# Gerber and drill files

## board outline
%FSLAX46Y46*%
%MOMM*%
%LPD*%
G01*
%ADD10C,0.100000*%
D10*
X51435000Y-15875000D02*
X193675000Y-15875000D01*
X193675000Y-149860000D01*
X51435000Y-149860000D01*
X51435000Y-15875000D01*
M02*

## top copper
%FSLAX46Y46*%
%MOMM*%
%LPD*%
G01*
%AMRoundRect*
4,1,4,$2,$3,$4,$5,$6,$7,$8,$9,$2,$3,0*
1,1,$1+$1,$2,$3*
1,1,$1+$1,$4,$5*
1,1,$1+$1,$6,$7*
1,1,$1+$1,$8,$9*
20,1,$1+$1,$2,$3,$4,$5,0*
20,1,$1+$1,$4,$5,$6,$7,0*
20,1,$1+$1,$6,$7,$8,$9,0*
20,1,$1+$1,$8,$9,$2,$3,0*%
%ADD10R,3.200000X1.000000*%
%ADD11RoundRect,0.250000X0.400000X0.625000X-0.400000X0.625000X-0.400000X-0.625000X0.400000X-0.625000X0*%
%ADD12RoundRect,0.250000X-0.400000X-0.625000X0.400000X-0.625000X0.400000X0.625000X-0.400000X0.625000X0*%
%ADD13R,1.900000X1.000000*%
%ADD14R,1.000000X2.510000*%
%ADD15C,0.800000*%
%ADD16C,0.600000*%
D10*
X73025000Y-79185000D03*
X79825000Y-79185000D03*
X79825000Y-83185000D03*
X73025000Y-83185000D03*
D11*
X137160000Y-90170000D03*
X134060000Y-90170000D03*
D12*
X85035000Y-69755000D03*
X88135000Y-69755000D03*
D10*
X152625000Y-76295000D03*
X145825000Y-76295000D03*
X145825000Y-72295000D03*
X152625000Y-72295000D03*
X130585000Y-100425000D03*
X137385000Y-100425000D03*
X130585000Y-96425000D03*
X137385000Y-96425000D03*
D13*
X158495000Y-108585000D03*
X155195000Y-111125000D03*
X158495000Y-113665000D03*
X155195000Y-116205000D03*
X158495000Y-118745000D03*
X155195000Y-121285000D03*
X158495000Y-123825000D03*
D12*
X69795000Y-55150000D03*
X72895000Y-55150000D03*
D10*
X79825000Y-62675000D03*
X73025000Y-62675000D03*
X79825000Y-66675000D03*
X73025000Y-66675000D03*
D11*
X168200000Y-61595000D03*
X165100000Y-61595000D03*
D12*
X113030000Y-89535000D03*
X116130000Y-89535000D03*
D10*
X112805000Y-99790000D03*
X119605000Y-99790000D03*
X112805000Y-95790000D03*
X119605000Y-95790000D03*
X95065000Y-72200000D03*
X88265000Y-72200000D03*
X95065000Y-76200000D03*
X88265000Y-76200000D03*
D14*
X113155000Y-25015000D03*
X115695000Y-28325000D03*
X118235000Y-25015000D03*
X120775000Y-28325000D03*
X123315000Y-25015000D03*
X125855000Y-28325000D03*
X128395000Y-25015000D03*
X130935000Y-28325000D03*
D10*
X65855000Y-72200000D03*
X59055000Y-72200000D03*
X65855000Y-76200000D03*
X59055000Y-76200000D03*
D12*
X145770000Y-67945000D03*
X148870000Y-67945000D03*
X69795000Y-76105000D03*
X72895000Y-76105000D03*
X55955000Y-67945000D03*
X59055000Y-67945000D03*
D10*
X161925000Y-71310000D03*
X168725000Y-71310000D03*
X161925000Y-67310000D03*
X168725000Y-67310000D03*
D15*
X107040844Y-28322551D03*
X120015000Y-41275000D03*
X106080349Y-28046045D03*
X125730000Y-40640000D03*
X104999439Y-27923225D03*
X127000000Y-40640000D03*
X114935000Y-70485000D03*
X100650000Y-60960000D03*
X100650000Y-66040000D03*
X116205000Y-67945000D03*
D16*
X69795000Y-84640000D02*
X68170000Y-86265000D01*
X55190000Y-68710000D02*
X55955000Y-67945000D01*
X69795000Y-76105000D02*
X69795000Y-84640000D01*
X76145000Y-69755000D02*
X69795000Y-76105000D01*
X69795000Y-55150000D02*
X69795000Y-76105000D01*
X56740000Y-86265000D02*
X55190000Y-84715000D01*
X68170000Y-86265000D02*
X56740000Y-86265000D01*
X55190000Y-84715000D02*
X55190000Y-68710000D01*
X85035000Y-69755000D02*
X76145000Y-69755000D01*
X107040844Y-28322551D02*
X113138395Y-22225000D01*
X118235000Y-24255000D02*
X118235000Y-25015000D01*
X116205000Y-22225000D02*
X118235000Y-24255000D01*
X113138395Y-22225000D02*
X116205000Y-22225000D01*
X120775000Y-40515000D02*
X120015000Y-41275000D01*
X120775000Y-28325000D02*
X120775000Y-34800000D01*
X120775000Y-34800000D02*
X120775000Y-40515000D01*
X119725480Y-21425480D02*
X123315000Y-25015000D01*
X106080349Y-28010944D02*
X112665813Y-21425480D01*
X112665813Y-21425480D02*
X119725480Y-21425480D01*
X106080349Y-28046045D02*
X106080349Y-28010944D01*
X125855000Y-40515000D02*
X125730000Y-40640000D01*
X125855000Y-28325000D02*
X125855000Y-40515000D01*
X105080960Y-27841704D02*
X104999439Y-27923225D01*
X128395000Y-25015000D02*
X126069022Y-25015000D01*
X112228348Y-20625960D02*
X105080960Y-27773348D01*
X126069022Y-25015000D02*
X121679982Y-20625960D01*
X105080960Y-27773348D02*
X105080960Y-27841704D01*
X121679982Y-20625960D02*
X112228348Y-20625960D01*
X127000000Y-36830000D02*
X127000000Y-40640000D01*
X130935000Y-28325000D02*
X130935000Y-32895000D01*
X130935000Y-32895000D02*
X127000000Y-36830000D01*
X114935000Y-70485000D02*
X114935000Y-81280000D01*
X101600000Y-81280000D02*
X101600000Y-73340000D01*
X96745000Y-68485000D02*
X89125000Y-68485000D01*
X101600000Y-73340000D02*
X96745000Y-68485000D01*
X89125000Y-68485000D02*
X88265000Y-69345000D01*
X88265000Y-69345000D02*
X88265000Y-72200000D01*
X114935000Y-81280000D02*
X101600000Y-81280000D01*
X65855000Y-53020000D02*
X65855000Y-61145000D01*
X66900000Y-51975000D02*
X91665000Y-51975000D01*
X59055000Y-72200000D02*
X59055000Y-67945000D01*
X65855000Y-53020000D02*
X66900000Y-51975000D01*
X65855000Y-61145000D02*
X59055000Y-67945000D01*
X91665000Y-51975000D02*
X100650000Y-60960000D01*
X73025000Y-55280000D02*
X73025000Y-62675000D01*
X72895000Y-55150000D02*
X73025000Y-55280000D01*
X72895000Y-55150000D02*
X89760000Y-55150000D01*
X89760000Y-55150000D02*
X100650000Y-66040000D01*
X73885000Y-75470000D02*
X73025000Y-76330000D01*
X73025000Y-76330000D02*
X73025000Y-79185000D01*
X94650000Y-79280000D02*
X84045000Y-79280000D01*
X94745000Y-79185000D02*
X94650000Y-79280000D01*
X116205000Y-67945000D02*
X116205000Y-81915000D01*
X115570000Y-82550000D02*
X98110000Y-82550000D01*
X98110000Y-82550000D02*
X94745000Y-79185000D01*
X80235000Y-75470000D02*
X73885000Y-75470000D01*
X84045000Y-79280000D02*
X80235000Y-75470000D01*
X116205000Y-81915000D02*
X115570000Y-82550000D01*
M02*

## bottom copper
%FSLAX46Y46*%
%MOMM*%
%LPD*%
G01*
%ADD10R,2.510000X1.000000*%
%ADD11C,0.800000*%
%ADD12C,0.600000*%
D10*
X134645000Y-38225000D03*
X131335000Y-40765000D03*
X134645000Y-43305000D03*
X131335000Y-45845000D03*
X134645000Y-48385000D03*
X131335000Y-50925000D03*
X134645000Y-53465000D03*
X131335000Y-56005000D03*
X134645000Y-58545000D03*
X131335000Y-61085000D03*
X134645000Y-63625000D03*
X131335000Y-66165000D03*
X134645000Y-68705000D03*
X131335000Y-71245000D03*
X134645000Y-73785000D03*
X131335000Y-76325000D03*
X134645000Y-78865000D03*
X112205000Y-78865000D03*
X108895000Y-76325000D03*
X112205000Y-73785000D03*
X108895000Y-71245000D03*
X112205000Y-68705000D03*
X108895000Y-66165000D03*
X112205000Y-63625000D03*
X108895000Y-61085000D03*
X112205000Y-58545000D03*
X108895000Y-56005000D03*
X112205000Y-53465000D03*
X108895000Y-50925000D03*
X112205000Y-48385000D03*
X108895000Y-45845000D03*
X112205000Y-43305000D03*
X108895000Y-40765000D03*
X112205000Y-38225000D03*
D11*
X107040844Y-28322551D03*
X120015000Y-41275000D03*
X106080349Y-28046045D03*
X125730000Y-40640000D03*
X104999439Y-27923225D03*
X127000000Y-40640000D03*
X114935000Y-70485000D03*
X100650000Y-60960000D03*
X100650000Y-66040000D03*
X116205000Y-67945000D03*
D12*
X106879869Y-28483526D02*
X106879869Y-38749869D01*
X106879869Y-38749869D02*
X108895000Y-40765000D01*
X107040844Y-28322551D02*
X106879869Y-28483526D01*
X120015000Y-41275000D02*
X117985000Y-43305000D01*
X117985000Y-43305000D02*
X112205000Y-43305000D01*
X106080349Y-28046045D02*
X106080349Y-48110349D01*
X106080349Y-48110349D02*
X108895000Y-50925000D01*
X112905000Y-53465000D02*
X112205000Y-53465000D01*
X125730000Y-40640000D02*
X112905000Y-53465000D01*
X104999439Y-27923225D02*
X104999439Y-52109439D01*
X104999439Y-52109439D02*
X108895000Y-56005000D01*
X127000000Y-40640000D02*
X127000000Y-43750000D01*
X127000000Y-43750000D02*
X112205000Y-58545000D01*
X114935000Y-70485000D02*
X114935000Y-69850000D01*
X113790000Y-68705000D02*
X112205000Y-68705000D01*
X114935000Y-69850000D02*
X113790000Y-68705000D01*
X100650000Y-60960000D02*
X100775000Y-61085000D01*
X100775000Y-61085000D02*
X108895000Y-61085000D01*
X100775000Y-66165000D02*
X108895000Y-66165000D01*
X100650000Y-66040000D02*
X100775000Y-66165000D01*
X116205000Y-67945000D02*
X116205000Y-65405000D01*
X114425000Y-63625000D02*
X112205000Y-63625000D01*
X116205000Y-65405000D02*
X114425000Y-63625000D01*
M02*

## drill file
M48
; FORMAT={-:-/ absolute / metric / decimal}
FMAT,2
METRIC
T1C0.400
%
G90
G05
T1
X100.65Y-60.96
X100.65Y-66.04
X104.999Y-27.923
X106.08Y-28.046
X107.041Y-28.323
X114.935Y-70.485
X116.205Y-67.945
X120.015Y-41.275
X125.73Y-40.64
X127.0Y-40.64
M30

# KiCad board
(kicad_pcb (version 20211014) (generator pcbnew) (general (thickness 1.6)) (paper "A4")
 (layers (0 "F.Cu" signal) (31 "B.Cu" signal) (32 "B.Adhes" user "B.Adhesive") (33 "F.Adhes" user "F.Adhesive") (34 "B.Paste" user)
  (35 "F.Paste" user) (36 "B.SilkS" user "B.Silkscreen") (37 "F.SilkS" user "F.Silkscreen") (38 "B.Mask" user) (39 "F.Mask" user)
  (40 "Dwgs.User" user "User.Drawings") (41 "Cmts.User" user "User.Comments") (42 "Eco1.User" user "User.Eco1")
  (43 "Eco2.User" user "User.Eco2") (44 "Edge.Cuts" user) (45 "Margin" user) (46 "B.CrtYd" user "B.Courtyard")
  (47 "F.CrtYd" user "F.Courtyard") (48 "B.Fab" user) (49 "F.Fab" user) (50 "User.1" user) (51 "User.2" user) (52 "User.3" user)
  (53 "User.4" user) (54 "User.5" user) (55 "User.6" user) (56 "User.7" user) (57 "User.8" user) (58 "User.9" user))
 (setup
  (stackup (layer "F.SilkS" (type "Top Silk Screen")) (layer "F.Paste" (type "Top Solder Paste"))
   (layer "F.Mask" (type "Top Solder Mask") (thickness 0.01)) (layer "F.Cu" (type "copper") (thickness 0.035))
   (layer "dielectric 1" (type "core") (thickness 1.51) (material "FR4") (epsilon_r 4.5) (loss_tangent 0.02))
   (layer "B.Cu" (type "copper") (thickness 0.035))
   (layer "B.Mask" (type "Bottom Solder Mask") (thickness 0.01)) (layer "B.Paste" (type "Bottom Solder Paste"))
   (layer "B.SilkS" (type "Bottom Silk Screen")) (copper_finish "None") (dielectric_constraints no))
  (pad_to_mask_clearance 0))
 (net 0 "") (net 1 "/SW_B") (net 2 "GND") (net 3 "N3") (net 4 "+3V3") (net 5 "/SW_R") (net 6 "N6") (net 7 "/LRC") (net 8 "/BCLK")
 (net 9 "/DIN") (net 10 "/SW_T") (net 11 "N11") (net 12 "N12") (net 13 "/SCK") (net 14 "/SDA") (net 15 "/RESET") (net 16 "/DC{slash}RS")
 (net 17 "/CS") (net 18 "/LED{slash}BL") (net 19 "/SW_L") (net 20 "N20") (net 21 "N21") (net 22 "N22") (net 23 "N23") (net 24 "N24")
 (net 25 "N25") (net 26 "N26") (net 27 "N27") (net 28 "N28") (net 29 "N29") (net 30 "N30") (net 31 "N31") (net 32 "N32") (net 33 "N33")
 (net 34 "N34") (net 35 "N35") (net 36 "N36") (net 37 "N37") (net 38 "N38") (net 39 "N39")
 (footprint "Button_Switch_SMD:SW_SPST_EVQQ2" (layer "F.Cu") (at 76.425 81.185)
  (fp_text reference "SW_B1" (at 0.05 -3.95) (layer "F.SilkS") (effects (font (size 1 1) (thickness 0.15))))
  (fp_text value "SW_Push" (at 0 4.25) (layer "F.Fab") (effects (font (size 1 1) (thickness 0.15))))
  (pad "1" smd rect (at -3.4 -2) (size 3.2 1) (layers "F.Cu" "F.Paste" "F.Mask") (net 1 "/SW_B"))
  (pad "1" smd rect (at 3.4 -2) (size 3.2 1) (layers "F.Cu" "F.Paste" "F.Mask") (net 1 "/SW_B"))
  (pad "2" smd rect (at 3.4 2) (size 3.2 1) (layers "F.Cu" "F.Paste" "F.Mask") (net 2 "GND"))
  (pad "2" smd rect (at -3.4 2) (size 3.2 1) (layers "F.Cu" "F.Paste" "F.Mask") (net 2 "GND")))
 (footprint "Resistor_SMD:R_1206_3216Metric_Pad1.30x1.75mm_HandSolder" (layer "F.Cu") (at 135.61 90.17 180)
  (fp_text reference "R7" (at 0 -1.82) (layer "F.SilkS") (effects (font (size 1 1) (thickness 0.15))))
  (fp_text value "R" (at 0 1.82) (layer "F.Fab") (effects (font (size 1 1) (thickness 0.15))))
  (pad "1" smd roundrect (at -1.55 0 180) (size 1.3 1.75) (layers "F.Cu" "F.Paste" "F.Mask") (roundrect_rratio 0.192308) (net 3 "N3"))
  (pad "2" smd roundrect (at 1.55 0 180) (size 1.3 1.75) (layers "F.Cu" "F.Paste" "F.Mask") (roundrect_rratio 0.192308) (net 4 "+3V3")))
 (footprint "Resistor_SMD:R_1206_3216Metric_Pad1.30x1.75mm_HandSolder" (layer "F.Cu") (at 86.585 69.755)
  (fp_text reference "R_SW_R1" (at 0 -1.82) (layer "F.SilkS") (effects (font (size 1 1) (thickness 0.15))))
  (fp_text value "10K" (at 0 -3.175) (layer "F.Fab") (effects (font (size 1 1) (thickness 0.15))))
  (pad "1" smd roundrect (at -1.55 0) (size 1.3 1.75) (layers "F.Cu" "F.Paste" "F.Mask") (roundrect_rratio 0.192308) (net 4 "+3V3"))
  (pad "2" smd roundrect (at 1.55 0) (size 1.3 1.75) (layers "F.Cu" "F.Paste" "F.Mask") (roundrect_rratio 0.192308) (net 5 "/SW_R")))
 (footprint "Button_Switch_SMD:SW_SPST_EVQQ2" (layer "F.Cu") (at 149.225 74.295 180)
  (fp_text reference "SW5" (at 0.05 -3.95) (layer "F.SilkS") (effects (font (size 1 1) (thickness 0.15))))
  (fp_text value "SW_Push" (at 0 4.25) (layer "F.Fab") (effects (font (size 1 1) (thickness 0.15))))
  (pad "1" smd rect (at -3.4 -2 180) (size 3.2 1) (layers "F.Cu" "F.Paste" "F.Mask") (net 2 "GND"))
  (pad "1" smd rect (at 3.4 -2 180) (size 3.2 1) (layers "F.Cu" "F.Paste" "F.Mask") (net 2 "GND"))
  (pad "2" smd rect (at 3.4 2 180) (size 3.2 1) (layers "F.Cu" "F.Paste" "F.Mask") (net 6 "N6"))
  (pad "2" smd rect (at -3.4 2 180) (size 3.2 1) (layers "F.Cu" "F.Paste" "F.Mask") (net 6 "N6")))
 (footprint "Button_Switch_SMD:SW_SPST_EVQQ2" (layer "F.Cu") (at 133.985 98.425 180)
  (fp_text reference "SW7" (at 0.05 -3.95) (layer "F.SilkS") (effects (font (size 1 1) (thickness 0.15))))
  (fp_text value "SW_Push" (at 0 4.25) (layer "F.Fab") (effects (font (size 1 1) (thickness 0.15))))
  (pad "1" smd rect (at 3.4 -2 180) (size 3.2 1) (layers "F.Cu" "F.Paste" "F.Mask") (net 2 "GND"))
  (pad "1" smd rect (at -3.4 -2 180) (size 3.2 1) (layers "F.Cu" "F.Paste" "F.Mask") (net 2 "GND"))
  (pad "2" smd rect (at 3.4 2 180) (size 3.2 1) (layers "F.Cu" "F.Paste" "F.Mask") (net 3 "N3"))
  (pad "2" smd rect (at -3.4 2 180) (size 3.2 1) (layers "F.Cu" "F.Paste" "F.Mask") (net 3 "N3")))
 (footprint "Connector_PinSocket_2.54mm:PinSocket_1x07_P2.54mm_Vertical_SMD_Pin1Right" (layer "F.Cu") (at 156.845 116.205)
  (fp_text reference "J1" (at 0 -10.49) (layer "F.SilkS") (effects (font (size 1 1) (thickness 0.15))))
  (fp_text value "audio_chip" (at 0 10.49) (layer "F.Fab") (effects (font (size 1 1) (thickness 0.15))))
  (pad "1" smd rect (at 1.65 -7.62) (size 1.9 1) (layers "F.Cu" "F.Paste" "F.Mask") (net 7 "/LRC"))
  (pad "2" smd rect (at -1.65 -5.08) (size 1.9 1) (layers "F.Cu" "F.Paste" "F.Mask") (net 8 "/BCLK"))
  (pad "3" smd rect (at 1.65 -2.54) (size 1.9 1) (layers "F.Cu" "F.Paste" "F.Mask") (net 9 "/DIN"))
  (pad "4" smd rect (at -1.65 0) (size 1.9 1) (layers "F.Cu" "F.Paste" "F.Mask") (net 2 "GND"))
  (pad "5" smd rect (at 1.65 2.54) (size 1.9 1) (layers "F.Cu" "F.Paste" "F.Mask") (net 2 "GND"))
  (pad "6" smd rect (at -1.65 5.08) (size 1.9 1) (layers "F.Cu" "F.Paste" "F.Mask") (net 2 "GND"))
  (pad "7" smd rect (at 1.65 7.62) (size 1.9 1) (layers "F.Cu" "F.Paste" "F.Mask") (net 4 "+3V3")))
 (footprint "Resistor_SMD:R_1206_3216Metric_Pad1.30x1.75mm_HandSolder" (layer "F.Cu") (at 71.345 55.15)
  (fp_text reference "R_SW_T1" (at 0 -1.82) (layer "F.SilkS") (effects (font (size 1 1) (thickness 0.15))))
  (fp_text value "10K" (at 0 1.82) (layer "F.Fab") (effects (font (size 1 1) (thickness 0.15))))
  (pad "1" smd roundrect (at -1.55 0) (size 1.3 1.75) (layers "F.Cu" "F.Paste" "F.Mask") (roundrect_rratio 0.192308) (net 4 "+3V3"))
  (pad "2" smd roundrect (at 1.55 0) (size 1.3 1.75) (layers "F.Cu" "F.Paste" "F.Mask") (roundrect_rratio 0.192308) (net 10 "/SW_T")))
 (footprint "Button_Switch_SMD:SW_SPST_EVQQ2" (layer "F.Cu") (at 76.425 64.675)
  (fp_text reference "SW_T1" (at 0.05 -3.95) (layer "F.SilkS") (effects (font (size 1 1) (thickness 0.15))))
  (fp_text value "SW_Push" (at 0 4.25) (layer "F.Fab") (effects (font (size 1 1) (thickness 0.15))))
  (pad "1" smd rect (at 3.4 -2) (size 3.2 1) (layers "F.Cu" "F.Paste" "F.Mask") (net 10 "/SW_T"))
  (pad "1" smd rect (at -3.4 -2) (size 3.2 1) (layers "F.Cu" "F.Paste" "F.Mask") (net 10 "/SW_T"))
  (pad "2" smd rect (at 3.4 2) (size 3.2 1) (layers "F.Cu" "F.Paste" "F.Mask") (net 2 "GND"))
  (pad "2" smd rect (at -3.4 2) (size 3.2 1) (layers "F.Cu" "F.Paste" "F.Mask") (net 2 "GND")))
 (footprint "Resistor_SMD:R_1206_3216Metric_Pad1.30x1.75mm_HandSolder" (layer "F.Cu") (at 166.65 61.595 180)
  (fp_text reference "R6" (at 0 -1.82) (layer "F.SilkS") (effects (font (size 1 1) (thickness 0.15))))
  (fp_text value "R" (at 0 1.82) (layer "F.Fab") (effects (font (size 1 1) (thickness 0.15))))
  (pad "1" smd roundrect (at -1.55 0 180) (size 1.3 1.75) (layers "F.Cu" "F.Paste" "F.Mask") (roundrect_rratio 0.192308) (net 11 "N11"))
  (pad "2" smd roundrect (at 1.55 0 180) (size 1.3 1.75) (layers "F.Cu" "F.Paste" "F.Mask") (roundrect_rratio 0.192308) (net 4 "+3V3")))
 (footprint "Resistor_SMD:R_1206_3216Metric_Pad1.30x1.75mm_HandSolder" (layer "F.Cu") (at 114.58 89.535)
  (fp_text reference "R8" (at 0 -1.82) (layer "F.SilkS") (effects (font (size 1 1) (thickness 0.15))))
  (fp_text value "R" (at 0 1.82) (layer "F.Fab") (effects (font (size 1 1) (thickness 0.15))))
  (pad "1" smd roundrect (at -1.55 0) (size 1.3 1.75) (layers "F.Cu" "F.Paste" "F.Mask") (roundrect_rratio 0.192308) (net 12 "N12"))
  (pad "2" smd roundrect (at 1.55 0) (size 1.3 1.75) (layers "F.Cu" "F.Paste" "F.Mask") (roundrect_rratio 0.192308) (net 4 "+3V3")))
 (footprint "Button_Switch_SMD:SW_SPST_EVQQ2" (layer "F.Cu") (at 116.205 97.79 180)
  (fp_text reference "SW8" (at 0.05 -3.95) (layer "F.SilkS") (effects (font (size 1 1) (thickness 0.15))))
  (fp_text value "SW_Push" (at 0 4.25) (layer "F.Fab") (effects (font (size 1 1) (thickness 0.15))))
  (pad "1" smd rect (at 3.4 -2 180) (size 3.2 1) (layers "F.Cu" "F.Paste" "F.Mask") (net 2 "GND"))
  (pad "1" smd rect (at -3.4 -2 180) (size 3.2 1) (layers "F.Cu" "F.Paste" "F.Mask") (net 2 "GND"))
  (pad "2" smd rect (at 3.4 2 180) (size 3.2 1) (layers "F.Cu" "F.Paste" "F.Mask") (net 12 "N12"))
  (pad "2" smd rect (at -3.4 2 180) (size 3.2 1) (layers "F.Cu" "F.Paste" "F.Mask") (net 12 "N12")))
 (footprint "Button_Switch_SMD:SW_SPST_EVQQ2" (layer "F.Cu") (at 91.665 74.2)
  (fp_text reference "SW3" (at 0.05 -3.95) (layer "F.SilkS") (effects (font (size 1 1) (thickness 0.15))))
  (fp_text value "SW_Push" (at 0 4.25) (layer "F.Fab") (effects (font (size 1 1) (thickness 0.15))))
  (pad "1" smd rect (at 3.4 -2) (size 3.2 1) (layers "F.Cu" "F.Paste" "F.Mask") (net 5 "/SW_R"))
  (pad "1" smd rect (at -3.4 -2) (size 3.2 1) (layers "F.Cu" "F.Paste" "F.Mask") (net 5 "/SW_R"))
  (pad "2" smd rect (at 3.4 2) (size 3.2 1) (layers "F.Cu" "F.Paste" "F.Mask") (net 2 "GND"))
  (pad "2" smd rect (at -3.4 2) (size 3.2 1) (layers "F.Cu" "F.Paste" "F.Mask") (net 2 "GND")))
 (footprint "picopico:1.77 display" (layer "F.Cu") (at 121.92 22.86 90)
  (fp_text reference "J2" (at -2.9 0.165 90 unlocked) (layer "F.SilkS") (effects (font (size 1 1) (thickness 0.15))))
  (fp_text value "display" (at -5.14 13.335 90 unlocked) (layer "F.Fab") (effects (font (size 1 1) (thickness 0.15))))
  (pad "1" smd rect (at -2.155 -8.765 90) (size 2.51 1) (layers "F.Cu" "F.Paste" "F.Mask") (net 2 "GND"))
  (pad "2" smd rect (at -5.465 -6.225 90) (size 2.51 1) (layers "F.Cu" "F.Paste" "F.Mask") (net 4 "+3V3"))
  (pad "3" smd rect (at -2.155 -3.685 90) (size 2.51 1) (layers "F.Cu" "F.Paste" "F.Mask") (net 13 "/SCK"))
  (pad "4" smd rect (at -5.465 -1.145 90) (size 2.51 1) (layers "F.Cu" "F.Paste" "F.Mask") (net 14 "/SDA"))
  (pad "5" smd rect (at -2.155 1.395 90) (size 2.51 1) (layers "F.Cu" "F.Paste" "F.Mask") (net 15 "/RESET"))
  (pad "6" smd rect (at -5.465 3.935 90) (size 2.51 1) (layers "F.Cu" "F.Paste" "F.Mask") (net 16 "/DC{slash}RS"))
  (pad "7" smd rect (at -2.155 6.475 90) (size 2.51 1) (layers "F.Cu" "F.Paste" "F.Mask") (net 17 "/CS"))
  (pad "8" smd rect (at -5.465 9.015 90) (size 2.51 1) (layers "F.Cu" "F.Paste" "F.Mask") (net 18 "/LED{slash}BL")))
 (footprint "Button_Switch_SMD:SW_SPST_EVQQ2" (layer "F.Cu") (at 62.455 74.2)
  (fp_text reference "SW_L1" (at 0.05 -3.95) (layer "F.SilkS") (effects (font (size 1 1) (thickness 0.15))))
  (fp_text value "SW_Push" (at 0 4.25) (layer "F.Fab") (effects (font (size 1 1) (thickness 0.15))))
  (pad "1" smd rect (at 3.4 -2) (size 3.2 1) (layers "F.Cu" "F.Paste" "F.Mask") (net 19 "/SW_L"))
  (pad "1" smd rect (at -3.4 -2) (size 3.2 1) (layers "F.Cu" "F.Paste" "F.Mask") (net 19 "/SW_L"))
  (pad "2" smd rect (at 3.4 2) (size 3.2 1) (layers "F.Cu" "F.Paste" "F.Mask") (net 2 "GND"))
  (pad "2" smd rect (at -3.4 2) (size 3.2 1) (layers "F.Cu" "F.Paste" "F.Mask") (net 2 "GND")))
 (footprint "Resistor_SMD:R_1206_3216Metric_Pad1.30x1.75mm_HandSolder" (layer "F.Cu") (at 147.32 67.945)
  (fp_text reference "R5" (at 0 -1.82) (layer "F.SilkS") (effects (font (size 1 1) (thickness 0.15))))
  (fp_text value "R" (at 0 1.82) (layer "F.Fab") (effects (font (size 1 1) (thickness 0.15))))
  (pad "1" smd roundrect (at -1.55 0) (size 1.3 1.75) (layers "F.Cu" "F.Paste" "F.Mask") (roundrect_rratio 0.192308) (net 6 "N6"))
  (pad "2" smd roundrect (at 1.55 0) (size 1.3 1.75) (layers "F.Cu" "F.Paste" "F.Mask") (roundrect_rratio 0.192308) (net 4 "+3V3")))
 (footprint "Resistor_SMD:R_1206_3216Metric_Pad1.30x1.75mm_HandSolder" (layer "F.Cu") (at 71.345 76.105)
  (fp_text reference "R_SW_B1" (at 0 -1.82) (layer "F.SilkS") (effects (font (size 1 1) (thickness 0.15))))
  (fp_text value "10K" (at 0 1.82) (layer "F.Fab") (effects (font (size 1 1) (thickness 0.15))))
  (pad "1" smd roundrect (at -1.55 0) (size 1.3 1.75) (layers "F.Cu" "F.Paste" "F.Mask") (roundrect_rratio 0.192308) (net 4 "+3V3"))
  (pad "2" smd roundrect (at 1.55 0) (size 1.3 1.75) (layers "F.Cu" "F.Paste" "F.Mask") (roundrect_rratio 0.192308) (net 1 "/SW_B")))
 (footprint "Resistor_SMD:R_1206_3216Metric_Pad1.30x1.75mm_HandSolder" (layer "F.Cu") (at 57.505 67.945)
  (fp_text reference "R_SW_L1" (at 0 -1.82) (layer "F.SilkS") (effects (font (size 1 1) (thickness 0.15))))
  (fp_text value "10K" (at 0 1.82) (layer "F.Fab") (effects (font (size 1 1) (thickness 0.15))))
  (pad "1" smd roundrect (at -1.55 0) (size 1.3 1.75) (layers "F.Cu" "F.Paste" "F.Mask") (roundrect_rratio 0.192308) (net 4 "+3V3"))
  (pad "2" smd roundrect (at 1.55 0) (size 1.3 1.75) (layers "F.Cu" "F.Paste" "F.Mask") (roundrect_rratio 0.192308) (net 19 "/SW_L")))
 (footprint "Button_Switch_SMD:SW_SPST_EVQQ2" (layer "F.Cu") (at 165.325 69.31 180)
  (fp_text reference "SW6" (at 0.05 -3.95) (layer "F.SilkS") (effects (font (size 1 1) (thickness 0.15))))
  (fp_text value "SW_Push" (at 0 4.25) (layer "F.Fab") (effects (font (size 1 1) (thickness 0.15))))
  (pad "1" smd rect (at 3.4 -2 180) (size 3.2 1) (layers "F.Cu" "F.Paste" "F.Mask") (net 2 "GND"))
  (pad "1" smd rect (at -3.4 -2 180) (size 3.2 1) (layers "F.Cu" "F.Paste" "F.Mask") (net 2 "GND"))
  (pad "2" smd rect (at 3.4 2 180) (size 3.2 1) (layers "F.Cu" "F.Paste" "F.Mask") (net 11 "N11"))
  (pad "2" smd rect (at -3.4 2 180) (size 3.2 1) (layers "F.Cu" "F.Paste" "F.Mask") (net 11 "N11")))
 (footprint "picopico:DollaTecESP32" (layer "B.Cu") (at 121.92 57.785 180)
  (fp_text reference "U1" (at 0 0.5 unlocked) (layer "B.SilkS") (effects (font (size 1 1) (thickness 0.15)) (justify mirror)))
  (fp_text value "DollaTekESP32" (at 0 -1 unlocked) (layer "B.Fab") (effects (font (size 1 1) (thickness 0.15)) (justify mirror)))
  (pad "1" smd rect (at -12.725 19.56 180) (size 2.51 1) (layers "B.Cu" "B.Paste" "B.Mask") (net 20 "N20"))
  (pad "2" smd rect (at -9.415 17.02 180) (size 2.51 1) (layers "B.Cu" "B.Paste" "B.Mask") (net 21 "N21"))
  (pad "3" smd rect (at -12.725 14.48 180) (size 2.51 1) (layers "B.Cu" "B.Paste" "B.Mask") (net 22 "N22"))
  (pad "4" smd rect (at -9.415 11.94 180) (size 2.51 1) (layers "B.Cu" "B.Paste" "B.Mask") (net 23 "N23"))
  (pad "5" smd rect (at -12.725 9.4 180) (size 2.51 1) (layers "B.Cu" "B.Paste" "B.Mask") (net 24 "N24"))
  (pad "6" smd rect (at -9.415 6.86 180) (size 2.51 1) (layers "B.Cu" "B.Paste" "B.Mask") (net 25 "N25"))
  (pad "7" smd rect (at -12.725 4.32 180) (size 2.51 1) (layers "B.Cu" "B.Paste" "B.Mask") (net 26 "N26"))
  (pad "8" smd rect (at -9.415 1.78 180) (size 2.51 1) (layers "B.Cu" "B.Paste" "B.Mask") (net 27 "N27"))
  (pad "9" smd rect (at -12.725 -0.76 180) (size 2.51 1) (layers "B.Cu" "B.Paste" "B.Mask") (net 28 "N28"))
  (pad "10" smd rect (at -9.415 -3.3 180) (size 2.51 1) (layers "B.Cu" "B.Paste" "B.Mask") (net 9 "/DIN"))
  (pad "11" smd rect (at -12.725 -5.84 180) (size 2.51 1) (layers "B.Cu" "B.Paste" "B.Mask") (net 8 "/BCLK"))
  (pad "12" smd rect (at -9.415 -8.38 180) (size 2.51 1) (layers "B.Cu" "B.Paste" "B.Mask") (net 7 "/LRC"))
  (pad "13" smd rect (at -12.725 -10.92 180) (size 2.51 1) (layers "B.Cu" "B.Paste" "B.Mask") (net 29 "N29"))
  (pad "14" smd rect (at -9.415 -13.46 180) (size 2.51 1) (layers "B.Cu" "B.Paste" "B.Mask") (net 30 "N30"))
  (pad "15" smd rect (at -12.725 -16 180) (size 2.51 1) (layers "B.Cu" "B.Paste" "B.Mask") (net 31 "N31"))
  (pad "16" smd rect (at -9.415 -18.54 180) (size 2.51 1) (layers "B.Cu" "B.Paste" "B.Mask") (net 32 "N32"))
  (pad "17" smd rect (at -12.725 -21.08 180) (size 2.51 1) (layers "B.Cu" "B.Paste" "B.Mask") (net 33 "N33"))
  (pad "18" smd rect (at 9.715 -21.08 180) (size 2.51 1) (layers "B.Cu" "B.Paste" "B.Mask") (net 4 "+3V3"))
  (pad "19" smd rect (at 13.025 -18.54 180) (size 2.51 1) (layers "B.Cu" "B.Paste" "B.Mask") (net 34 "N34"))
  (pad "20" smd rect (at 9.715 -16 180) (size 2.51 1) (layers "B.Cu" "B.Paste" "B.Mask") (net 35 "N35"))
  (pad "21" smd rect (at 13.025 -13.46 180) (size 2.51 1) (layers "B.Cu" "B.Paste" "B.Mask") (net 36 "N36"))
  (pad "22" smd rect (at 9.715 -10.92 180) (size 2.51 1) (layers "B.Cu" "B.Paste" "B.Mask") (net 5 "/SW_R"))
  (pad "23" smd rect (at 13.025 -8.38 180) (size 2.51 1) (layers "B.Cu" "B.Paste" "B.Mask") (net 10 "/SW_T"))
  (pad "24" smd rect (at 9.715 -5.84 180) (size 2.51 1) (layers "B.Cu" "B.Paste" "B.Mask") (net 1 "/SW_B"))
  (pad "25" smd rect (at 13.025 -3.3 180) (size 2.51 1) (layers "B.Cu" "B.Paste" "B.Mask") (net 19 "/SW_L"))
  (pad "26" smd rect (at 9.715 -0.76 180) (size 2.51 1) (layers "B.Cu" "B.Paste" "B.Mask") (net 18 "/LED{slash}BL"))
  (pad "27" smd rect (at 13.025 1.78 180) (size 2.51 1) (layers "B.Cu" "B.Paste" "B.Mask") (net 17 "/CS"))
  (pad "28" smd rect (at 9.715 4.32 180) (size 2.51 1) (layers "B.Cu" "B.Paste" "B.Mask") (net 16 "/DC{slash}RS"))
  (pad "29" smd rect (at 13.025 6.86 180) (size 2.51 1) (layers "B.Cu" "B.Paste" "B.Mask") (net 15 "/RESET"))
  (pad "30" smd rect (at 9.715 9.4 180) (size 2.51 1) (layers "B.Cu" "B.Paste" "B.Mask") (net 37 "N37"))
  (pad "31" smd rect (at 13.025 11.94 180) (size 2.51 1) (layers "B.Cu" "B.Paste" "B.Mask") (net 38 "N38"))
  (pad "32" smd rect (at 9.715 14.48 180) (size 2.51 1) (layers "B.Cu" "B.Paste" "B.Mask") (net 14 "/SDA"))
  (pad "33" smd rect (at 13.025 17.02 180) (size 2.51 1) (layers "B.Cu" "B.Paste" "B.Mask") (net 13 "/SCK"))
  (pad "34" smd rect (at 9.715 19.56 180) (size 2.51 1) (layers "B.Cu" "B.Paste" "B.Mask") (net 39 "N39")))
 (gr_rect (start 51.435 15.875) (end 193.675 149.86) (layer "Edge.Cuts") (width 0.1) (fill none))
 (segment (start 69.795 84.64) (end 68.17 86.265) (width 0.6) (layer "F.Cu") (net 4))
 (segment (start 55.19 68.71) (end 55.955 67.945) (width 0.6) (layer "F.Cu") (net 4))
 (segment (start 69.795 76.105) (end 69.795 84.64) (width 0.6) (layer "F.Cu") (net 4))
 (segment (start 76.145 69.755) (end 69.795 76.105) (width 0.6) (layer "F.Cu") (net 4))
 (segment (start 69.795 55.15) (end 69.795 76.105) (width 0.6) (layer "F.Cu") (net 4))
 (segment (start 56.74 86.265) (end 55.19 84.715) (width 0.6) (layer "F.Cu") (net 4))
 (segment (start 68.17 86.265) (end 56.74 86.265) (width 0.6) (layer "F.Cu") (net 4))
 (segment (start 55.19 84.715) (end 55.19 68.71) (width 0.6) (layer "F.Cu") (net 4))
 (segment (start 85.035 69.755) (end 76.145 69.755) (width 0.6) (layer "F.Cu") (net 4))
 (segment (start 107.040844 28.322551) (end 113.138395 22.225) (width 0.6) (layer "F.Cu") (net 13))
 (segment (start 118.235 24.255) (end 118.235 25.015) (width 0.6) (layer "F.Cu") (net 13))
 (segment (start 116.205 22.225) (end 118.235 24.255) (width 0.6) (layer "F.Cu") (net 13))
 (segment (start 113.138395 22.225) (end 116.205 22.225) (width 0.6) (layer "F.Cu") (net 13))
 (via (at 107.040844 28.322551) (size 0.8) (drill 0.4) (layers "F.Cu" "B.Cu") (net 13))
 (segment (start 106.879869 28.483526) (end 106.879869 38.749869) (width 0.6) (layer "B.Cu") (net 13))
 (segment (start 106.879869 38.749869) (end 108.895 40.765) (width 0.6) (layer "B.Cu") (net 13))
 (segment (start 107.040844 28.322551) (end 106.879869 28.483526) (width 0.6) (layer "B.Cu") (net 13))
 (segment (start 120.775 40.515) (end 120.015 41.275) (width 0.6) (layer "F.Cu") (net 14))
 (segment (start 120.775 28.325) (end 120.775 34.8) (width 0.6) (layer "F.Cu") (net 14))
 (segment (start 120.775 34.8) (end 120.775 40.515) (width 0.6) (layer "F.Cu") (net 14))
 (via (at 120.015 41.275) (size 0.8) (drill 0.4) (layers "F.Cu" "B.Cu") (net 14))
 (segment (start 120.015 41.275) (end 117.985 43.305) (width 0.6) (layer "B.Cu") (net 14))
 (segment (start 117.985 43.305) (end 112.205 43.305) (width 0.6) (layer "B.Cu") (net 14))
 (segment (start 119.72548 21.42548) (end 123.315 25.015) (width 0.6) (layer "F.Cu") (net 15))
 (segment (start 106.080349 28.010944) (end 112.665813 21.42548) (width 0.6) (layer "F.Cu") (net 15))
 (segment (start 112.665813 21.42548) (end 119.72548 21.42548) (width 0.6) (layer "F.Cu") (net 15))
 (segment (start 106.080349 28.046045) (end 106.080349 28.010944) (width 0.6) (layer "F.Cu") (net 15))
 (via (at 106.080349 28.046045) (size 0.8) (drill 0.4) (layers "F.Cu" "B.Cu") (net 15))
 (segment (start 106.080349 28.046045) (end 106.080349 48.110349) (width 0.6) (layer "B.Cu") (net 15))
 (segment (start 106.080349 48.110349) (end 108.895 50.925) (width 0.6) (layer "B.Cu") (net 15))
 (segment (start 125.855 40.515) (end 125.73 40.64) (width 0.6) (layer "F.Cu") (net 16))
 (segment (start 125.855 28.325) (end 125.855 40.515) (width 0.6) (layer "F.Cu") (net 16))
 (via (at 125.73 40.64) (size 0.8) (drill 0.4) (layers "F.Cu" "B.Cu") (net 16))
 (segment (start 112.905 53.465) (end 112.205 53.465) (width 0.6) (layer "B.Cu") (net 16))
 (segment (start 125.73 40.64) (end 112.905 53.465) (width 0.6) (layer "B.Cu") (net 16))
 (segment (start 105.08096 27.841704) (end 104.999439 27.923225) (width 0.6) (layer "F.Cu") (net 17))
 (segment (start 128.395 25.015) (end 126.069022 25.015) (width 0.6) (layer "F.Cu") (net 17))
 (segment (start 112.228348 20.62596) (end 105.08096 27.773348) (width 0.6) (layer "F.Cu") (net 17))
 (segment (start 126.069022 25.015) (end 121.679982 20.62596) (width 0.6) (layer "F.Cu") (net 17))
 (segment (start 105.08096 27.773348) (end 105.08096 27.841704) (width 0.6) (layer "F.Cu") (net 17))
 (segment (start 121.679982 20.62596) (end 112.228348 20.62596) (width 0.6) (layer "F.Cu") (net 17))
 (via (at 104.999439 27.923225) (size 0.8) (drill 0.4) (layers "F.Cu" "B.Cu") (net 17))
 (segment (start 104.999439 27.923225) (end 104.999439 52.109439) (width 0.6) (layer "B.Cu") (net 17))
 (segment (start 104.999439 52.109439) (end 108.895 56.005) (width 0.6) (layer "B.Cu") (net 17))
 (segment (start 127 36.83) (end 127 40.64) (width 0.6) (layer "F.Cu") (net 18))
 (segment (start 130.935 28.325) (end 130.935 32.895) (width 0.6) (layer "F.Cu") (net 18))
 (segment (start 130.935 32.895) (end 127 36.83) (width 0.6) (layer "F.Cu") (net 18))
 (via (at 127 40.64) (size 0.8) (drill 0.4) (layers "F.Cu" "B.Cu") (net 18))
 (segment (start 127 40.64) (end 127 43.75) (width 0.6) (layer "B.Cu") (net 18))
 (segment (start 127 43.75) (end 112.205 58.545) (width 0.6) (layer "B.Cu") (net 18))
 (segment (start 114.935 70.485) (end 114.935 81.28) (width 0.6) (layer "F.Cu") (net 5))
 (segment (start 101.6 81.28) (end 101.6 73.34) (width 0.6) (layer "F.Cu") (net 5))
 (segment (start 96.745 68.485) (end 89.125 68.485) (width 0.6) (layer "F.Cu") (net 5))
 (segment (start 101.6 73.34) (end 96.745 68.485) (width 0.6) (layer "F.Cu") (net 5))
 (segment (start 89.125 68.485) (end 88.265 69.345) (width 0.6) (layer "F.Cu") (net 5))
 (segment (start 88.265 69.345) (end 88.265 72.2) (width 0.6) (layer "F.Cu") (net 5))
 (segment (start 114.935 81.28) (end 101.6 81.28) (width 0.6) (layer "F.Cu") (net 5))
 (via (at 114.935 70.485) (size 0.8) (drill 0.4) (layers "F.Cu" "B.Cu") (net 5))
 (segment (start 114.935 70.485) (end 114.935 69.85) (width 0.6) (layer "B.Cu") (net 5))
 (segment (start 113.79 68.705) (end 112.205 68.705) (width 0.6) (layer "B.Cu") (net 5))
 (segment (start 114.935 69.85) (end 113.79 68.705) (width 0.6) (layer "B.Cu") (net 5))
 (segment (start 65.855 53.02) (end 65.855 61.145) (width 0.6) (layer "F.Cu") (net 19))
 (segment (start 66.9 51.975) (end 91.665 51.975) (width 0.6) (layer "F.Cu") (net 19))
 (segment (start 59.055 72.2) (end 59.055 67.945) (width 0.6) (layer "F.Cu") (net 19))
 (segment (start 65.855 53.02) (end 66.9 51.975) (width 0.6) (layer "F.Cu") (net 19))
 (segment (start 65.855 61.145) (end 59.055 67.945) (width 0.6) (layer "F.Cu") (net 19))
 (segment (start 91.665 51.975) (end 100.65 60.96) (width 0.6) (layer "F.Cu") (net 19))
 (via (at 100.65 60.96) (size 0.8) (drill 0.4) (layers "F.Cu" "B.Cu") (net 19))
 (segment (start 100.65 60.96) (end 100.775 61.085) (width 0.6) (layer "B.Cu") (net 19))
 (segment (start 100.775 61.085) (end 108.895 61.085) (width 0.6) (layer "B.Cu") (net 19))
 (segment (start 73.025 55.28) (end 73.025 62.675) (width 0.6) (layer "F.Cu") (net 10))
 (segment (start 72.895 55.15) (end 73.025 55.28) (width 0.6) (layer "F.Cu") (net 10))
 (segment (start 72.895 55.15) (end 89.76 55.15) (width 0.6) (layer "F.Cu") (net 10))
 (segment (start 89.76 55.15) (end 100.65 66.04) (width 0.6) (layer "F.Cu") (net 10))
 (via (at 100.65 66.04) (size 0.8) (drill 0.4) (layers "F.Cu" "B.Cu") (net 10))
 (segment (start 100.775 66.165) (end 108.895 66.165) (width 0.6) (layer "B.Cu") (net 10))
 (segment (start 100.65 66.04) (end 100.775 66.165) (width 0.6) (layer "B.Cu") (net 10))
 (segment (start 73.885 75.47) (end 73.025 76.33) (width 0.6) (layer "F.Cu") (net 1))
 (segment (start 73.025 76.33) (end 73.025 79.185) (width 0.6) (layer "F.Cu") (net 1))
 (segment (start 94.65 79.28) (end 84.045 79.28) (width 0.6) (layer "F.Cu") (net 1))
 (segment (start 94.745 79.185) (end 94.65 79.28) (width 0.6) (layer "F.Cu") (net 1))
 (segment (start 116.205 67.945) (end 116.205 81.915) (width 0.6) (layer "F.Cu") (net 1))
 (segment (start 115.57 82.55) (end 98.11 82.55) (width 0.6) (layer "F.Cu") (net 1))
 (segment (start 98.11 82.55) (end 94.745 79.185) (width 0.6) (layer "F.Cu") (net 1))
 (segment (start 80.235 75.47) (end 73.885 75.47) (width 0.6) (layer "F.Cu") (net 1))
 (segment (start 84.045 79.28) (end 80.235 75.47) (width 0.6) (layer "F.Cu") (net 1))
 (segment (start 116.205 81.915) (end 115.57 82.55) (width 0.6) (layer "F.Cu") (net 1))
 (via (at 116.205 67.945) (size 0.8) (drill 0.4) (layers "F.Cu" "B.Cu") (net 1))
 (segment (start 116.205 67.945) (end 116.205 65.405) (width 0.6) (layer "B.Cu") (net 1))
 (segment (start 114.425 63.625) (end 112.205 63.625) (width 0.6) (layer "B.Cu") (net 1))
 (segment (start 116.205 65.405) (end 114.425 63.625) (width 0.6) (layer "B.Cu") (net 1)))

